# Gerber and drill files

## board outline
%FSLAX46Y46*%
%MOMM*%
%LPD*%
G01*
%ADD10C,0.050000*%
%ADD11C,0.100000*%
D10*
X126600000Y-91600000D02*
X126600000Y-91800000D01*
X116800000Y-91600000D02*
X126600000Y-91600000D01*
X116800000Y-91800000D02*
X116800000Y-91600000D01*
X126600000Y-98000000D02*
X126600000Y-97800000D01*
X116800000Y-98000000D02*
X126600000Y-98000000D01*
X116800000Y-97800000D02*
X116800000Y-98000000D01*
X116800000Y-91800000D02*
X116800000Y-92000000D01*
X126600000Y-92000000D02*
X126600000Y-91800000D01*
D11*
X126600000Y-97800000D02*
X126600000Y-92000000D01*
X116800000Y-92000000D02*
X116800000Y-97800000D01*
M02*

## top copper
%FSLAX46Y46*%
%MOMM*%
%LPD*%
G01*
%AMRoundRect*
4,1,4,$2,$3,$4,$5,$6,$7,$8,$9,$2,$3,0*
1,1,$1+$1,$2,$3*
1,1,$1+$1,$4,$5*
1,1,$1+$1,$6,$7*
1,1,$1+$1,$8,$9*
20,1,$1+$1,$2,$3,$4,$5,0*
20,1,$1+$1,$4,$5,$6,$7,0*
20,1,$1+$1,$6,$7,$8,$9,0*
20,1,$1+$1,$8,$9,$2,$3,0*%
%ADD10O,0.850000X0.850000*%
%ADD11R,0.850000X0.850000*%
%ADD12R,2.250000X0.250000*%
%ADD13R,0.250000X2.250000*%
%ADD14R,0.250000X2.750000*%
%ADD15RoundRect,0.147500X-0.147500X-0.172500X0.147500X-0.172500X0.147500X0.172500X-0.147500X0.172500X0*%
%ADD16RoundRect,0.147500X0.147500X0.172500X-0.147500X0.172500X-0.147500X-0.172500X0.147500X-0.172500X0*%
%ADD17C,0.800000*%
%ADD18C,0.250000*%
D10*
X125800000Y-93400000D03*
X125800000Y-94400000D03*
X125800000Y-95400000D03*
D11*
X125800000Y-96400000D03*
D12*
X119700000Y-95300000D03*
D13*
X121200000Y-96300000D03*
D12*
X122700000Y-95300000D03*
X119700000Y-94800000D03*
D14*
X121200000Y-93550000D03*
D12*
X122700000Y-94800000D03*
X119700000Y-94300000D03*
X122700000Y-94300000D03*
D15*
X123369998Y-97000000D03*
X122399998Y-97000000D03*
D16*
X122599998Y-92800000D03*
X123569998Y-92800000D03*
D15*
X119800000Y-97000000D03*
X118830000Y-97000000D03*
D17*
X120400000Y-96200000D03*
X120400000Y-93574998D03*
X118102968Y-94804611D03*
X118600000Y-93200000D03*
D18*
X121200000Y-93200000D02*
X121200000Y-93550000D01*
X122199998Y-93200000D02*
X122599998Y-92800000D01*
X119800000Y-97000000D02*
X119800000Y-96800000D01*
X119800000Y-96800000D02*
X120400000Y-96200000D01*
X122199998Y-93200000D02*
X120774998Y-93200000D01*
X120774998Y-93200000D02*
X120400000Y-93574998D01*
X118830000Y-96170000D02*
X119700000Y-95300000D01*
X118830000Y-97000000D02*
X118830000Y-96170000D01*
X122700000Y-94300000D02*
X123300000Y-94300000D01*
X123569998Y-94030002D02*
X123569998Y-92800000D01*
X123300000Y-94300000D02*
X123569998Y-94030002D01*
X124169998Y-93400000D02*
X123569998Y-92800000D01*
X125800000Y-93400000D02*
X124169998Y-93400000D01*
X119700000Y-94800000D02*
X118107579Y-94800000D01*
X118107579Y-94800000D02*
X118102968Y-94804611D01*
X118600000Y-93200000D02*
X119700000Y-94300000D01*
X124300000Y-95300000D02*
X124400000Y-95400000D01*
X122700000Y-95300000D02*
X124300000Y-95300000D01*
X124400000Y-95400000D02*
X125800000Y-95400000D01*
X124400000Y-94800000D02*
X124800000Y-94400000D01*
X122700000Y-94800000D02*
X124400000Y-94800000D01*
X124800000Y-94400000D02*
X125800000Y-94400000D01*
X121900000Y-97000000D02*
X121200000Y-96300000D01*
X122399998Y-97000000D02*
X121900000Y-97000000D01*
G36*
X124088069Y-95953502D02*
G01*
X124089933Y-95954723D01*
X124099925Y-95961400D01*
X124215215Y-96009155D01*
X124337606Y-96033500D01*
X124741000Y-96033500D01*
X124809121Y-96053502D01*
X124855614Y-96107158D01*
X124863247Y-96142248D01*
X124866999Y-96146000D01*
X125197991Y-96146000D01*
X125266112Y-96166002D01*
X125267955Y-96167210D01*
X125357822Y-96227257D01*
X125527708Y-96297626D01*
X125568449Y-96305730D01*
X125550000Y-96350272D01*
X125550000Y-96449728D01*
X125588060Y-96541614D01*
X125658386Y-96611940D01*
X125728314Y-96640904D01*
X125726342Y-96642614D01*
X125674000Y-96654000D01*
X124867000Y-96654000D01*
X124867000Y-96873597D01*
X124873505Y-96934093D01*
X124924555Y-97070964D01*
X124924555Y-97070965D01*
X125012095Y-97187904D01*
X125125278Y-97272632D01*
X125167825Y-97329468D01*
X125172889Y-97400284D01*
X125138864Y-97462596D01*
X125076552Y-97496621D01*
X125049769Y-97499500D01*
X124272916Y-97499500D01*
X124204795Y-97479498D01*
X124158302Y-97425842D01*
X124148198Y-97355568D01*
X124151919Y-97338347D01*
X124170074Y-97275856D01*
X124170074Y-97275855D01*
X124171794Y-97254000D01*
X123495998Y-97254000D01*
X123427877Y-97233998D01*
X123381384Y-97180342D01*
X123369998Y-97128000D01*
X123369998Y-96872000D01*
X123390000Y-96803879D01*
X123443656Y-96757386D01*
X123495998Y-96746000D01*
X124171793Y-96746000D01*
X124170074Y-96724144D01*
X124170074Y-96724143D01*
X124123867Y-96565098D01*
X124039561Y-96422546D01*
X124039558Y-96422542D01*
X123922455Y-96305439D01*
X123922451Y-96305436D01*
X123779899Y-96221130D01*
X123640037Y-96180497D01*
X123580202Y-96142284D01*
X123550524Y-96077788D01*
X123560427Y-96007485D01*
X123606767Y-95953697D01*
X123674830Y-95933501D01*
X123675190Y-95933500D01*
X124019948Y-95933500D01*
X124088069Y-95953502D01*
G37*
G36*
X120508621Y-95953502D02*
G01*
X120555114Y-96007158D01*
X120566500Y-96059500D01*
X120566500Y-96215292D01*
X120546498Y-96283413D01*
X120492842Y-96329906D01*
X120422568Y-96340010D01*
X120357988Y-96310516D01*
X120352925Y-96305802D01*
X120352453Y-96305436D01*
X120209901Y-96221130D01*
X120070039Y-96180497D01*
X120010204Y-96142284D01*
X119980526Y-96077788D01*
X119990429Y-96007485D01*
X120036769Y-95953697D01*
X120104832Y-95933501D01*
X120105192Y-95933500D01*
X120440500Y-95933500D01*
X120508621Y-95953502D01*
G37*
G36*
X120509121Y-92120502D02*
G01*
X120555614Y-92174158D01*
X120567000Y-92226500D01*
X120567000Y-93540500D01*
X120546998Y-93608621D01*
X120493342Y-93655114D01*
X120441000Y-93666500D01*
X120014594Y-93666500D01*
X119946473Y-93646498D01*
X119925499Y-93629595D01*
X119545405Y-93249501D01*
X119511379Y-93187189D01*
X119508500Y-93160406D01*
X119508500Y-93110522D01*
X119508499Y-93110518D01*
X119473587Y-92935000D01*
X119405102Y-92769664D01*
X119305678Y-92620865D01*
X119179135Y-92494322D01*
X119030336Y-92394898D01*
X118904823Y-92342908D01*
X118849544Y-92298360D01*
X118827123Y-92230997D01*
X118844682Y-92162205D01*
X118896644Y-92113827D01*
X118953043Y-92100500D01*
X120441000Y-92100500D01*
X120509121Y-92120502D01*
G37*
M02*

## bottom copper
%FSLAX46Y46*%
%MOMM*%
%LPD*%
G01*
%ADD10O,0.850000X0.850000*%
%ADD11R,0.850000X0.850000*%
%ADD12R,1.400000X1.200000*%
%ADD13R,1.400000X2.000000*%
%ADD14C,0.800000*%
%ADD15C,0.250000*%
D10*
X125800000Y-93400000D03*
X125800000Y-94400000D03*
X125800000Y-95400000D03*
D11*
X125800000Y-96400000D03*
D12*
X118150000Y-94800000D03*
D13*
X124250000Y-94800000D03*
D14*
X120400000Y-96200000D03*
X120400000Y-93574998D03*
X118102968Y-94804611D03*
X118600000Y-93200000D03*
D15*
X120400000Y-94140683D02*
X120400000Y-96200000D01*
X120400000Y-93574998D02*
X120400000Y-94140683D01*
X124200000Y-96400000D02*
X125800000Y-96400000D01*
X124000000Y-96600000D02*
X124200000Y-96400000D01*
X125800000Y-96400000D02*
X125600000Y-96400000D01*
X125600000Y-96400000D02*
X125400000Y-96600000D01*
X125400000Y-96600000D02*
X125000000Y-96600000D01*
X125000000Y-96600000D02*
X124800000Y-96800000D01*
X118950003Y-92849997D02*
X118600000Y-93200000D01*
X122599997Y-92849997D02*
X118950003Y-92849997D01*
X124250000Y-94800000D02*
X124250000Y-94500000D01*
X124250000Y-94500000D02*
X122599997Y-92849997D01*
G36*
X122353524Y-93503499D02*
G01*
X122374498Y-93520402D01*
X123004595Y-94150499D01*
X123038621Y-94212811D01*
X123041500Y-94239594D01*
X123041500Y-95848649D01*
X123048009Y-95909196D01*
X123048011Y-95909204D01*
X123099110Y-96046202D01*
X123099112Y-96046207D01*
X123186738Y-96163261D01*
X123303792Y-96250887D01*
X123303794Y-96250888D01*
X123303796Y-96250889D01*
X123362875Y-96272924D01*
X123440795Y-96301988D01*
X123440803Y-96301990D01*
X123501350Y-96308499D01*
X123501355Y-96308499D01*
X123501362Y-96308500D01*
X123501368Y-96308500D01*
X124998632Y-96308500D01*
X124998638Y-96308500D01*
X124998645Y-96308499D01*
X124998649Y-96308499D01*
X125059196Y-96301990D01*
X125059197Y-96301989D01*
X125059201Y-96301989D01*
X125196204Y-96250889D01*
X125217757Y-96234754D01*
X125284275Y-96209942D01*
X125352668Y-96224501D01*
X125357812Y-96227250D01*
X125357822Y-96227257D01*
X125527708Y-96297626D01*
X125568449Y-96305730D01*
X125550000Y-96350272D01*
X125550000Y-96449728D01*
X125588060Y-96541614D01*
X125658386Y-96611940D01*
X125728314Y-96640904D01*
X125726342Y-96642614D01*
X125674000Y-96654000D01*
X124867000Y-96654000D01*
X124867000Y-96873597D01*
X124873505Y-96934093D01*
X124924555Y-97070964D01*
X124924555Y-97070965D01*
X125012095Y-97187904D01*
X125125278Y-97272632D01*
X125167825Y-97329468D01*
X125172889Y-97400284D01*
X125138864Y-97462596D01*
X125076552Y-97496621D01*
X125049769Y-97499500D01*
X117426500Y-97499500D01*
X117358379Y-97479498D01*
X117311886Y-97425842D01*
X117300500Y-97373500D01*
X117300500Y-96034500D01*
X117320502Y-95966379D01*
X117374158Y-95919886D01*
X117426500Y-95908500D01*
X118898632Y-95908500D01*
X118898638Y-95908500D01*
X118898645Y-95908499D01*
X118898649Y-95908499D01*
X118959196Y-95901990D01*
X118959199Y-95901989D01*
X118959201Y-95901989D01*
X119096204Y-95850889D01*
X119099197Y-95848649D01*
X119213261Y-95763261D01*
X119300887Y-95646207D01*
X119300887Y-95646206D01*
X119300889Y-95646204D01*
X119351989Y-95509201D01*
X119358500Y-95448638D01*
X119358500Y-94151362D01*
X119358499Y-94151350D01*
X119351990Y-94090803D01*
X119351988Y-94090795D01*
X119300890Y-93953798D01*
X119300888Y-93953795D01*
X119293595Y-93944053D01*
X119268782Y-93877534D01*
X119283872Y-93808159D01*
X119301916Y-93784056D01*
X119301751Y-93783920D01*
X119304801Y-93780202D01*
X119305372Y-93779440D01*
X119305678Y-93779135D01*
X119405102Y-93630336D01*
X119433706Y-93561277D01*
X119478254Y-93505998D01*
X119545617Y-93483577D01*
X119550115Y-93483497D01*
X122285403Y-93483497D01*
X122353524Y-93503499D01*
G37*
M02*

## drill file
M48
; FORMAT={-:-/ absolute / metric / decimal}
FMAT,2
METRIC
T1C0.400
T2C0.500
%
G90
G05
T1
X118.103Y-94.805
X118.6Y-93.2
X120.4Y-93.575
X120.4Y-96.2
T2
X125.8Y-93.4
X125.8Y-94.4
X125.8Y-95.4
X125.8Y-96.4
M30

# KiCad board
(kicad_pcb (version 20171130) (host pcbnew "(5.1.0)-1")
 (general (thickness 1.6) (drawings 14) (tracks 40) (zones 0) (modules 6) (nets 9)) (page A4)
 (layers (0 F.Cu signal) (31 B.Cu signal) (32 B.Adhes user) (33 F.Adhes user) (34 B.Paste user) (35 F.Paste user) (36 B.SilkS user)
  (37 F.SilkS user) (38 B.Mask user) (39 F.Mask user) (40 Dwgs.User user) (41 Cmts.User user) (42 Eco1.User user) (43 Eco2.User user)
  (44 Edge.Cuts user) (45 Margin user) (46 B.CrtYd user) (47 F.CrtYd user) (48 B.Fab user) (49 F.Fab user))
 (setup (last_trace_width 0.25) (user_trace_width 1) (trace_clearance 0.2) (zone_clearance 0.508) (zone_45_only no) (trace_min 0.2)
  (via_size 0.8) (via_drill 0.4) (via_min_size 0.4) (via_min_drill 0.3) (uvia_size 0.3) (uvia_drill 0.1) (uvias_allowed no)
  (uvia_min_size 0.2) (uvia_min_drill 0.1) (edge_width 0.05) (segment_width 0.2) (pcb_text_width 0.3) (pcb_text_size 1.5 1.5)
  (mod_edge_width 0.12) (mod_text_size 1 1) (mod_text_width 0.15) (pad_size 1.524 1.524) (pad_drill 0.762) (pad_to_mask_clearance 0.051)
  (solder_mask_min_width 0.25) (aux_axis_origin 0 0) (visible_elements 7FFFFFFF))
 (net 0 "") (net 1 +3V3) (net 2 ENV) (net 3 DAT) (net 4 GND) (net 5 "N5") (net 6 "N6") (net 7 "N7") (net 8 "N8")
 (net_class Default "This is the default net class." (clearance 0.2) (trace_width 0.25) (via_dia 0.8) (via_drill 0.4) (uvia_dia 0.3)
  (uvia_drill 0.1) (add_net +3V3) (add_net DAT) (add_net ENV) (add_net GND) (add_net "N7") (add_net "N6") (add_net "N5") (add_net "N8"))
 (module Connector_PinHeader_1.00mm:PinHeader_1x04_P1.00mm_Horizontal (layer B.Cu) (at 125.8 96.4)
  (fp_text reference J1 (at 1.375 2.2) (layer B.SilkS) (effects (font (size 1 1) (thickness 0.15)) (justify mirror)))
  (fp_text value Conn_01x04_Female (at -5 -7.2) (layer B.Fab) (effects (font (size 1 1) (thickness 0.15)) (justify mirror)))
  (pad 4 thru_hole oval (at 0 -3) (size 0.85 0.85) (drill 0.5) (layers *.Cu *.Mask) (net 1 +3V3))
  (pad 3 thru_hole oval (at 0 -2) (size 0.85 0.85) (drill 0.5) (layers *.Cu *.Mask) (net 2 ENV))
  (pad 2 thru_hole oval (at 0 -1) (size 0.85 0.85) (drill 0.5) (layers *.Cu *.Mask) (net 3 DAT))
  (pad 1 thru_hole rect (at 0 0) (size 0.85 0.85) (drill 0.5) (layers *.Cu *.Mask) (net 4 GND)))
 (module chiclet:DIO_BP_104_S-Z (layer B.Cu) (at 121.2 94.8)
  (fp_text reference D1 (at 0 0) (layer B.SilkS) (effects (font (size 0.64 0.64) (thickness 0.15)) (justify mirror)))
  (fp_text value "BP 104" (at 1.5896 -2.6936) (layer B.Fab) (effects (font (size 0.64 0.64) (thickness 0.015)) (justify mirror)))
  (pad 2 smd rect (at -3.05 0) (size 1.4 1.2) (layers B.Cu) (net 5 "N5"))
  (pad 1 smd rect (at 3.05 0) (size 1.4 2) (layers B.Cu) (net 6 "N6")))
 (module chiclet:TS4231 (layer F.Cu) (at 121.2 94.8 90)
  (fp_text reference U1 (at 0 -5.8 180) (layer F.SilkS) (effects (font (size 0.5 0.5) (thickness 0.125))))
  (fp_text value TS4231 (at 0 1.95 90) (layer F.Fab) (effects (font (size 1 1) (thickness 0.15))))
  (pad A1 smd rect (at -0.5 -1.5 90) (size 0.25 2.25) (layers F.Cu F.Paste F.Mask) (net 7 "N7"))
  (pad B1 smd rect (at -1.5 0 90) (size 2.25 0.25) (layers F.Cu F.Paste F.Mask) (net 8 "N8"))
  (pad C1 smd rect (at -0.5 1.5 90) (size 0.25 2.25) (layers F.Cu F.Paste F.Mask) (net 3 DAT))
  (pad A2 smd rect (at 0 -1.5 90) (size 0.25 2.25) (layers F.Cu F.Paste F.Mask) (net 5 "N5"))
  (pad B2 smd rect (at 1.25 0 90) (size 2.75 0.25) (layers F.Cu F.Paste F.Mask) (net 4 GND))
  (pad C2 smd rect (at 0 1.5 90) (size 0.25 2.25) (layers F.Cu F.Paste F.Mask) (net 2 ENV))
  (pad A3 smd rect (at 0.5 -1.5 90) (size 0.25 2.25) (layers F.Cu F.Paste F.Mask) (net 6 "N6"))
  (pad C3 smd rect (at 0.5 1.5 90) (size 0.25 2.25) (layers F.Cu F.Paste F.Mask) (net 1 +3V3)))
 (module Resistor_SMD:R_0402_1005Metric (layer F.Cu) (at 122.884998 97)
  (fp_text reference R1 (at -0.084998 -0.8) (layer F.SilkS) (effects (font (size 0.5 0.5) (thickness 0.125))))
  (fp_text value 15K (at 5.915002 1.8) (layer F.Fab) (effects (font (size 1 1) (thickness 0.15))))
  (pad 2 smd roundrect (at 0.485 0) (size 0.59 0.64) (layers F.Cu F.Paste F.Mask) (roundrect_rratio 0.25) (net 4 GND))
  (pad 1 smd roundrect (at -0.485 0) (size 0.59 0.64) (layers F.Cu F.Paste F.Mask) (roundrect_rratio 0.25) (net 8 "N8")))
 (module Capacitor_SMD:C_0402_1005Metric (layer F.Cu) (at 123.084998 92.8 180)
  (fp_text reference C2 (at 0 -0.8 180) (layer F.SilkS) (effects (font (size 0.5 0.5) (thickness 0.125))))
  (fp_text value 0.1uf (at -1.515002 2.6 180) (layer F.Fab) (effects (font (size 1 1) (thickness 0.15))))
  (pad 2 smd roundrect (at 0.485 0 180) (size 0.59 0.64) (layers F.Cu F.Paste F.Mask) (roundrect_rratio 0.25) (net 4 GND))
  (pad 1 smd roundrect (at -0.485 0 180) (size 0.59 0.64) (layers F.Cu F.Paste F.Mask) (roundrect_rratio 0.25) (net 1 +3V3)))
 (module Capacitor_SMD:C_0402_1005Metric (layer F.Cu) (at 119.315 97)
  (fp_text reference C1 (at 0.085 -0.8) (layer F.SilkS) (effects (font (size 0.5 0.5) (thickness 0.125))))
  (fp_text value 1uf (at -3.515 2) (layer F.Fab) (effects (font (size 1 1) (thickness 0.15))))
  (pad 2 smd roundrect (at 0.485 0) (size 0.59 0.64) (layers F.Cu F.Paste F.Mask) (roundrect_rratio 0.25) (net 4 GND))
  (pad 1 smd roundrect (at -0.485 0) (size 0.59 0.64) (layers F.Cu F.Paste F.Mask) (roundrect_rratio 0.25) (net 7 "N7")))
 (gr_line (start 126.6 91.6) (end 126.6 91.8) (layer Edge.Cuts) (width 0.05))
 (gr_line (start 116.8 91.6) (end 126.6 91.6) (layer Edge.Cuts) (width 0.05))
 (gr_line (start 116.8 91.8) (end 116.8 91.6) (layer Edge.Cuts) (width 0.05))
 (gr_line (start 126.6 98) (end 126.6 97.8) (layer Edge.Cuts) (width 0.05))
 (gr_line (start 116.8 98) (end 126.6 98) (layer Edge.Cuts) (width 0.05))
 (gr_line (start 116.8 97.8) (end 116.8 98) (layer Edge.Cuts) (width 0.05))
 (gr_line (start 116.8 91.8) (end 116.8 92) (layer Edge.Cuts) (width 0.05))
 (gr_line (start 126.6 92) (end 126.6 91.8) (layer Edge.Cuts) (width 0.05))
 (gr_line (start 126.6 97.8) (end 126.6 92) (layer Edge.Cuts) (width 0.1))
 (gr_line (start 116.8 92) (end 116.8 97.8) (layer Edge.Cuts) (width 0.1))
 (segment (start 121.2 93.2) (end 121.2 93.55) (width 0.25) (layer F.Cu) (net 4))
 (segment (start 122.199998 93.2) (end 122.599998 92.8) (width 0.25) (layer F.Cu) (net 4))
 (via (at 120.4 96.2) (size 0.8) (drill 0.4) (layers F.Cu B.Cu) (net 4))
 (segment (start 119.8 97) (end 119.8 96.8) (width 0.25) (layer F.Cu) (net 4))
 (segment (start 119.8 96.8) (end 120.4 96.2) (width 0.25) (layer F.Cu) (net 4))
 (via (at 120.4 93.574998) (size 0.8) (drill 0.4) (layers F.Cu B.Cu) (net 4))
 (segment (start 122.199998 93.2) (end 120.774998 93.2) (width 0.25) (layer F.Cu) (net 4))
 (segment (start 120.774998 93.2) (end 120.4 93.574998) (width 0.25) (layer F.Cu) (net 4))
 (segment (start 120.4 94.140683) (end 120.4 96.2) (width 0.25) (layer B.Cu) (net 4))
 (segment (start 120.4 93.574998) (end 120.4 94.140683) (width 0.25) (layer B.Cu) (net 4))
 (segment (start 124.2 96.4) (end 125.8 96.4) (width 0.25) (layer B.Cu) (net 4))
 (segment (start 124 96.6) (end 124.2 96.4) (width 0.25) (layer B.Cu) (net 4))
 (segment (start 125.8 96.4) (end 125.6 96.4) (width 0.25) (layer B.Cu) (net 4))
 (segment (start 125.6 96.4) (end 125.4 96.6) (width 0.25) (layer B.Cu) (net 4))
 (segment (start 125.4 96.6) (end 125 96.6) (width 0.25) (layer B.Cu) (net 4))
 (segment (start 125 96.6) (end 124.8 96.8) (width 0.25) (layer B.Cu) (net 4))
 (segment (start 118.83 96.17) (end 119.7 95.3) (width 0.25) (layer F.Cu) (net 7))
 (segment (start 118.83 97) (end 118.83 96.17) (width 0.25) (layer F.Cu) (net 7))
 (segment (start 122.7 94.3) (end 123.3 94.3) (width 0.25) (layer F.Cu) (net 1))
 (segment (start 123.569998 94.030002) (end 123.569998 92.8) (width 0.25) (layer F.Cu) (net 1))
 (segment (start 123.3 94.3) (end 123.569998 94.030002) (width 0.25) (layer F.Cu) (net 1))
 (segment (start 124.169998 93.4) (end 123.569998 92.8) (width 0.25) (layer F.Cu) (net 1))
 (segment (start 125.8 93.4) (end 124.169998 93.4) (width 0.25) (layer F.Cu) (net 1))
 (via (at 118.102968 94.804611) (size 0.8) (drill 0.4) (layers F.Cu B.Cu) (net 5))
 (segment (start 119.7 94.8) (end 118.107579 94.8) (width 0.25) (layer F.Cu) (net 5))
 (segment (start 118.107579 94.8) (end 118.102968 94.804611) (width 0.25) (layer F.Cu) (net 5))
 (via (at 118.6 93.2) (size 0.8) (drill 0.4) (layers F.Cu B.Cu) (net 6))
 (segment (start 118.950003 92.849997) (end 118.6 93.2) (width 0.25) (layer B.Cu) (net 6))
 (segment (start 122.599997 92.849997) (end 118.950003 92.849997) (width 0.25) (layer B.Cu) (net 6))
 (segment (start 124.25 94.8) (end 124.25 94.5) (width 0.25) (layer B.Cu) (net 6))
 (segment (start 124.25 94.5) (end 122.599997 92.849997) (width 0.25) (layer B.Cu) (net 6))
 (segment (start 118.6 93.2) (end 119.7 94.3) (width 0.25) (layer F.Cu) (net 6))
 (segment (start 124.3 95.3) (end 124.4 95.4) (width 0.25) (layer F.Cu) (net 3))
 (segment (start 122.7 95.3) (end 124.3 95.3) (width 0.25) (layer F.Cu) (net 3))
 (segment (start 124.4 95.4) (end 125.8 95.4) (width 0.25) (layer F.Cu) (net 3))
 (segment (start 124.4 94.8) (end 124.8 94.4) (width 0.25) (layer F.Cu) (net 2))
 (segment (start 122.7 94.8) (end 124.4 94.8) (width 0.25) (layer F.Cu) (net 2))
 (segment (start 124.8 94.4) (end 125.8 94.4) (width 0.25) (layer F.Cu) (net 2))
 (segment (start 121.9 97) (end 121.2 96.3) (width 0.25) (layer F.Cu) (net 8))
 (segment (start 122.399998 97) (end 121.9 97) (width 0.25) (layer F.Cu) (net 8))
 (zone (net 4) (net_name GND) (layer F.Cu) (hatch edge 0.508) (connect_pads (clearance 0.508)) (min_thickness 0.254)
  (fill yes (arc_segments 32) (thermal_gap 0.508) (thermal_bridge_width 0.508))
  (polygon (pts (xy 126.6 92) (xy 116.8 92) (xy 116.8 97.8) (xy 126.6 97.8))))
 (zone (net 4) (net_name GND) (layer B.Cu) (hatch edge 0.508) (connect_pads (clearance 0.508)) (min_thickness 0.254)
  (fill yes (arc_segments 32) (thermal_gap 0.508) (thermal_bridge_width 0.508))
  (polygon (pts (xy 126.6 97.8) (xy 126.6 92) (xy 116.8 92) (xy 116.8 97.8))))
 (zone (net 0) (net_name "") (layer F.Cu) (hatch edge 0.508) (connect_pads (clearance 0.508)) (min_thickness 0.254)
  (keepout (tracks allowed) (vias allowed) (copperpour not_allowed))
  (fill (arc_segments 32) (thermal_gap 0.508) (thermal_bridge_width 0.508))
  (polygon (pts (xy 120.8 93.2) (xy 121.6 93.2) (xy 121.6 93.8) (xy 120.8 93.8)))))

